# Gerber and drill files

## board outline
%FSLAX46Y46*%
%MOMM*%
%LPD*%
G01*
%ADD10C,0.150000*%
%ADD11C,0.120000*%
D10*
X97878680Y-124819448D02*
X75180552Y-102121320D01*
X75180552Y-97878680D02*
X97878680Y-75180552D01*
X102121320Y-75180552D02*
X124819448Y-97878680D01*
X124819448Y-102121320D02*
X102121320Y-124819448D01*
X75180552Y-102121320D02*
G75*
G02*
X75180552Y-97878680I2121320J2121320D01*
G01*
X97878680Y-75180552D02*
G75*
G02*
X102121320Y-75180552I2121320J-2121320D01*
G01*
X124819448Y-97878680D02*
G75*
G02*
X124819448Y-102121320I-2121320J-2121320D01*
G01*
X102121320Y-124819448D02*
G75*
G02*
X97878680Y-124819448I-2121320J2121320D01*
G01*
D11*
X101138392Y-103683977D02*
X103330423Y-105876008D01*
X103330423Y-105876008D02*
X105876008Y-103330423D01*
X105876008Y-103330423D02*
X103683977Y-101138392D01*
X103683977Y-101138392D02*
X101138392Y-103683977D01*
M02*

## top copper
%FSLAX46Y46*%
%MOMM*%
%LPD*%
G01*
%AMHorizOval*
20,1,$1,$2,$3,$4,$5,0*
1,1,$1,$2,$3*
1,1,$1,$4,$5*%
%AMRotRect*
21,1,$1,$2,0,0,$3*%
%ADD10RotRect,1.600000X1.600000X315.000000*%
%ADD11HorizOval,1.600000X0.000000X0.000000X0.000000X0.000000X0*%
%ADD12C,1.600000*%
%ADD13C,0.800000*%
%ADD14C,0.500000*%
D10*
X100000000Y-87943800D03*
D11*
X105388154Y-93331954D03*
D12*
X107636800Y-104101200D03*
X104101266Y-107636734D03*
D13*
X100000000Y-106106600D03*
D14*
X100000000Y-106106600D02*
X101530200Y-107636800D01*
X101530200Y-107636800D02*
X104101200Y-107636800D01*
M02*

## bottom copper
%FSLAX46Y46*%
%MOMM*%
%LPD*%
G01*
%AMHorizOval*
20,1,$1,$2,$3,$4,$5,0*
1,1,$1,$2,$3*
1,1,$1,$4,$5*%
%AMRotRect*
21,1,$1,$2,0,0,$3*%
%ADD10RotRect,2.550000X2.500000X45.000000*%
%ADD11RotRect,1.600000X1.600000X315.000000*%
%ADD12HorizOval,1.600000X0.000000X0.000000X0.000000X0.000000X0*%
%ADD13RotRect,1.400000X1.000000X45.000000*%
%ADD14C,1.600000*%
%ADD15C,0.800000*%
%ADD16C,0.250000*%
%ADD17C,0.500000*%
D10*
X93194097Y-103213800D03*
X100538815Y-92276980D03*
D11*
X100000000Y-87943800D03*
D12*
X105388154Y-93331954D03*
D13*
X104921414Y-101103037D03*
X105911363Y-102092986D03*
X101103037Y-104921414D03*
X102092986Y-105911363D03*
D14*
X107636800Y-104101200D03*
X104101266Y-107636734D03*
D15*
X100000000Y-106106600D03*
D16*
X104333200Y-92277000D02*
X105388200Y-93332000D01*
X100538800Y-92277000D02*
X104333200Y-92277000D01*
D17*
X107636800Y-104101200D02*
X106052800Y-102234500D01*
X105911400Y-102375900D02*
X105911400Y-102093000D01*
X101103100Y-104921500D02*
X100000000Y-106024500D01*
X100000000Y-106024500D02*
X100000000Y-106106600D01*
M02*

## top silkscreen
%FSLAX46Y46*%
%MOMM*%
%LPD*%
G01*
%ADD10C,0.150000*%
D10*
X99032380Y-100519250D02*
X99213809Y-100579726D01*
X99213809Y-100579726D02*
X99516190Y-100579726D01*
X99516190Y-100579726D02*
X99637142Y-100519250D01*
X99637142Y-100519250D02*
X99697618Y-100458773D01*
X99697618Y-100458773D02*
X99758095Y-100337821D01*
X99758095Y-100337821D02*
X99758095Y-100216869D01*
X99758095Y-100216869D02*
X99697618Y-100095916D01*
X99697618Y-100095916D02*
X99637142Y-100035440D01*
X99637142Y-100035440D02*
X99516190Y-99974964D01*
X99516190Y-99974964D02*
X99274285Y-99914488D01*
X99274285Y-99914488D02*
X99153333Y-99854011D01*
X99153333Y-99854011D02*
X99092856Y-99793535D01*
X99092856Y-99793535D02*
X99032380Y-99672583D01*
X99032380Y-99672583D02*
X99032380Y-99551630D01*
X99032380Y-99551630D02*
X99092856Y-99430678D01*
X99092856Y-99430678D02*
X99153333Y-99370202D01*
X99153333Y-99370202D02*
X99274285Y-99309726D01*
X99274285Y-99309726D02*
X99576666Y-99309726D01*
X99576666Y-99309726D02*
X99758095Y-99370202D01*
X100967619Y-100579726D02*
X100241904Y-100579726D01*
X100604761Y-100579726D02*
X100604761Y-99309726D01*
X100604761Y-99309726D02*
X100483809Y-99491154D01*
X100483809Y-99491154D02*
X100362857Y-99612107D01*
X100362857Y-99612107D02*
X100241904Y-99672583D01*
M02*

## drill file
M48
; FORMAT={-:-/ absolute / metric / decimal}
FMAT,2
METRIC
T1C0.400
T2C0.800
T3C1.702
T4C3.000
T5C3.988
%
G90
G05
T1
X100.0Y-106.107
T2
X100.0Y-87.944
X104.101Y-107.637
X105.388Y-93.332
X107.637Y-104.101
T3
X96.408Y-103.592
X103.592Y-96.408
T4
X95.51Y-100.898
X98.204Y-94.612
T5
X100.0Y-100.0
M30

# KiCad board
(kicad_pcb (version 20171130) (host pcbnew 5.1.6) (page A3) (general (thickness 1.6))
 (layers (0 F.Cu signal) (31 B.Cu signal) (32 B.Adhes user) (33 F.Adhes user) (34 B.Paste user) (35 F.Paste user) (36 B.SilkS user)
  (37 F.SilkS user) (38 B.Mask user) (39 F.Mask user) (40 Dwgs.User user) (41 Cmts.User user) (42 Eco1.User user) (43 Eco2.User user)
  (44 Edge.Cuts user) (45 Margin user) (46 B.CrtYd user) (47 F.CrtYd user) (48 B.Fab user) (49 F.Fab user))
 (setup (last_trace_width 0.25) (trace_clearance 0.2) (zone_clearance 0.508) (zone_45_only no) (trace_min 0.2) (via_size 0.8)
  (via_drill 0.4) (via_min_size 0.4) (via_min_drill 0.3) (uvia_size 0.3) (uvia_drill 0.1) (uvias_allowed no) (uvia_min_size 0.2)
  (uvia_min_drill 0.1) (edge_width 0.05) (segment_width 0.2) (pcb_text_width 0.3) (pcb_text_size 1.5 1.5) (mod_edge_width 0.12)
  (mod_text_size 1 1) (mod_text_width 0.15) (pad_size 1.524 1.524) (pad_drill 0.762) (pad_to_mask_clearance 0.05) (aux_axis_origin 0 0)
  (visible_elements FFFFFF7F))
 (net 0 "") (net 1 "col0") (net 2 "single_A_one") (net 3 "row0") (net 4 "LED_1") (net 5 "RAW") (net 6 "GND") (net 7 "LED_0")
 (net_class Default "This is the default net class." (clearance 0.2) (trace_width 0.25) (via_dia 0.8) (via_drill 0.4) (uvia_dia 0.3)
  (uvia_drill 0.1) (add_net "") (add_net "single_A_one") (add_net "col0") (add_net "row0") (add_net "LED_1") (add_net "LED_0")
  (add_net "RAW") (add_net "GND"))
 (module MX (layer F.Cu) (at 100 100 45)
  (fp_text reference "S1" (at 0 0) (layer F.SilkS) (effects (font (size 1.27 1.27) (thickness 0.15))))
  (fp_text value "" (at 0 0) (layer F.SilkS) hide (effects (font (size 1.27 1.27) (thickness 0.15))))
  (pad "" np_thru_hole circle (at 0 0) (size 3.9878 3.9878) (drill 3.9878) (layers *.Cu *.Mask))
  (pad "" np_thru_hole circle (at 5.08 0) (size 1.7018 1.7018) (drill 1.7018) (layers *.Cu *.Mask))
  (pad "" np_thru_hole circle (at -5.08 0) (size 1.7018 1.7018) (drill 1.7018) (layers *.Cu *.Mask))
  (pad "" np_thru_hole circle (at 2.54 -5.08) (size 3 3) (drill 3) (layers *.Cu *.Mask))
  (pad "" np_thru_hole circle (at -3.81 -2.54) (size 3 3) (drill 3) (layers *.Cu *.Mask))
  (pad 1 smd rect (at -7.085 -2.54 45) (size 2.55 2.5) (layers B.Cu B.Paste B.Mask) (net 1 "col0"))
  (pad 2 smd rect (at 5.842 -5.08 45) (size 2.55 2.5) (layers B.Cu B.Paste B.Mask) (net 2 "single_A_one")))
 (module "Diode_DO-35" (layer "B.Cu") (at 100.0000 87.9438 315)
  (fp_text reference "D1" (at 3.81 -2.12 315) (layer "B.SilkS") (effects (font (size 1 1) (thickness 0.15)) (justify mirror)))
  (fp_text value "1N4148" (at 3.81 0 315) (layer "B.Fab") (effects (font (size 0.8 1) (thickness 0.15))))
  (pad 1 thru_hole rect (at 0 0 315) (size 1.6 1.6) (drill 0.8) (layers "*.Cu" "*.Mask") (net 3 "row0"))
  (pad 2 thru_hole oval (at 7.62 0 315) (size 1.6 1.6) (drill 0.8) (layers "*.Cu" "*.Mask") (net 2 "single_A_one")))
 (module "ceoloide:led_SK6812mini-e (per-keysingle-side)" (layer B.Cu) (at 103.5072 103.5072 45)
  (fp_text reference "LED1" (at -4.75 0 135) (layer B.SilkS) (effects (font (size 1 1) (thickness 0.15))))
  (pad 2 smd rect (at 2.70 -0.7 45) (size 1.4 1) (layers B.Cu B.Paste B.Mask) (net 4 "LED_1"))
  (pad 1 smd rect (at 2.70 0.7 45) (size 1.4 1) (layers B.Cu B.Paste B.Mask) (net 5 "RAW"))
  (pad 3 smd rect (at -2.70 -0.7 45) (size 1.4 1) (layers B.Cu B.Paste B.Mask) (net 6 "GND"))
  (pad 4 smd rect (at -2.70 0.7 45) (size 1.4 1) (layers B.Cu B.Paste B.Mask) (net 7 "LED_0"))
  (fp_line (start -1.8 -1.55) (end -1.8 1.55) (layer Edge.Cuts) (width 0.12))
  (fp_line (start -1.8 1.55) (end 1.8 1.55) (layer Edge.Cuts) (width 0.12))
  (fp_line (start 1.8 1.55) (end 1.8 -1.55) (layer Edge.Cuts) (width 0.12))
  (fp_line (start 1.8 -1.55) (end -1.8 -1.55) (layer Edge.Cuts) (width 0.12)))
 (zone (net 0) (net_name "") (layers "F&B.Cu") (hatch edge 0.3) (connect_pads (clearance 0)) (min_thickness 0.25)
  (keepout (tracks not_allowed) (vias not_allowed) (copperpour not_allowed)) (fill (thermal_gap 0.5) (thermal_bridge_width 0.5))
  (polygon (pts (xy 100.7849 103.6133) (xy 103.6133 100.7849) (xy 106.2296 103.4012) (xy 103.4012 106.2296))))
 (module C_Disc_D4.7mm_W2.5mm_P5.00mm (layer B.Cu) (at 107.6368 104.1012 225)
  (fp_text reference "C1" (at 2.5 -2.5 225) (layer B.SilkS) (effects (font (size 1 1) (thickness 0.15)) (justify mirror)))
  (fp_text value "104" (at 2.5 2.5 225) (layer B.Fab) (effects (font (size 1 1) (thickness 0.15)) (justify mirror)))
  (pad 1 thru_hole circle (at 0 0) (size 1.6 1.6) (drill 0.8) (layers *.Cu *.Mask) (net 5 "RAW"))
  (pad 2 thru_hole circle (at 5 0) (size 1.6 1.6) (drill 0.8) (layers *.Cu *.Mask) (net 6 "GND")))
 (segment (start 104.3332 92.2770) (end 105.3882 93.3320) (width 0.25) (layer "B.Cu") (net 2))
 (segment (start 100.5388 92.2770) (end 104.3332 92.2770) (width 0.25) (layer "B.Cu") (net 2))
 (segment (start 107.6368 104.1012) (end 106.0528 102.2345) (width 0.5) (layer "B.Cu") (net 5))
 (segment (start 105.9114 102.3759) (end 105.9114 102.0930) (width 0.5) (layer "B.Cu") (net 5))
 (segment (start 100.0000 106.1066) (end 101.5302 107.6368) (width 0.5) (layer "F.Cu") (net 6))
 (segment (start 101.5302 107.6368) (end 104.1012 107.6368) (width 0.5) (layer "F.Cu") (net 6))
 (via (at 100.0000 106.1066) (size 0.8) (drill 0.4) (layers "F.Cu" "B.Cu") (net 6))
 (segment (start 101.1031 104.9215) (end 100.0000 106.0245) (width 0.5) (layer "B.Cu") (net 6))
 (segment (start 100.0000 106.0245) (end 100.0000 106.1066) (width 0.5) (layer "B.Cu") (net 6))
 (gr_line (start 97.8786797 124.8194481) (end 75.1805519 102.1213203) (angle 90) (layer Edge.Cuts) (width 0.15))
 (gr_line (start 75.1805519 97.8786797) (end 97.8786797 75.1805519) (angle 90) (layer Edge.Cuts) (width 0.15))
 (gr_line (start 102.1213203 75.1805519) (end 124.8194481 97.8786797) (angle 90) (layer Edge.Cuts) (width 0.15))
 (gr_line (start 124.8194481 102.1213203) (end 102.1213203 124.8194481) (angle 90) (layer Edge.Cuts) (width 0.15))
 (gr_arc (start 77.30187219999999 100) (end 75.1805519 97.8786797) (angle -90) (layer Edge.Cuts) (width 0.15))
 (gr_arc (start 100 77.30187219999999) (end 102.1213203 75.1805519) (angle -90) (layer Edge.Cuts) (width 0.15))
 (gr_arc (start 122.69812780000001 100) (end 124.8194481 102.1213203) (angle -90) (layer Edge.Cuts) (width 0.15))
 (gr_arc (start 100 122.69812780000001) (end 97.8786797 124.8194481) (angle -90) (layer Edge.Cuts) (width 0.15)))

